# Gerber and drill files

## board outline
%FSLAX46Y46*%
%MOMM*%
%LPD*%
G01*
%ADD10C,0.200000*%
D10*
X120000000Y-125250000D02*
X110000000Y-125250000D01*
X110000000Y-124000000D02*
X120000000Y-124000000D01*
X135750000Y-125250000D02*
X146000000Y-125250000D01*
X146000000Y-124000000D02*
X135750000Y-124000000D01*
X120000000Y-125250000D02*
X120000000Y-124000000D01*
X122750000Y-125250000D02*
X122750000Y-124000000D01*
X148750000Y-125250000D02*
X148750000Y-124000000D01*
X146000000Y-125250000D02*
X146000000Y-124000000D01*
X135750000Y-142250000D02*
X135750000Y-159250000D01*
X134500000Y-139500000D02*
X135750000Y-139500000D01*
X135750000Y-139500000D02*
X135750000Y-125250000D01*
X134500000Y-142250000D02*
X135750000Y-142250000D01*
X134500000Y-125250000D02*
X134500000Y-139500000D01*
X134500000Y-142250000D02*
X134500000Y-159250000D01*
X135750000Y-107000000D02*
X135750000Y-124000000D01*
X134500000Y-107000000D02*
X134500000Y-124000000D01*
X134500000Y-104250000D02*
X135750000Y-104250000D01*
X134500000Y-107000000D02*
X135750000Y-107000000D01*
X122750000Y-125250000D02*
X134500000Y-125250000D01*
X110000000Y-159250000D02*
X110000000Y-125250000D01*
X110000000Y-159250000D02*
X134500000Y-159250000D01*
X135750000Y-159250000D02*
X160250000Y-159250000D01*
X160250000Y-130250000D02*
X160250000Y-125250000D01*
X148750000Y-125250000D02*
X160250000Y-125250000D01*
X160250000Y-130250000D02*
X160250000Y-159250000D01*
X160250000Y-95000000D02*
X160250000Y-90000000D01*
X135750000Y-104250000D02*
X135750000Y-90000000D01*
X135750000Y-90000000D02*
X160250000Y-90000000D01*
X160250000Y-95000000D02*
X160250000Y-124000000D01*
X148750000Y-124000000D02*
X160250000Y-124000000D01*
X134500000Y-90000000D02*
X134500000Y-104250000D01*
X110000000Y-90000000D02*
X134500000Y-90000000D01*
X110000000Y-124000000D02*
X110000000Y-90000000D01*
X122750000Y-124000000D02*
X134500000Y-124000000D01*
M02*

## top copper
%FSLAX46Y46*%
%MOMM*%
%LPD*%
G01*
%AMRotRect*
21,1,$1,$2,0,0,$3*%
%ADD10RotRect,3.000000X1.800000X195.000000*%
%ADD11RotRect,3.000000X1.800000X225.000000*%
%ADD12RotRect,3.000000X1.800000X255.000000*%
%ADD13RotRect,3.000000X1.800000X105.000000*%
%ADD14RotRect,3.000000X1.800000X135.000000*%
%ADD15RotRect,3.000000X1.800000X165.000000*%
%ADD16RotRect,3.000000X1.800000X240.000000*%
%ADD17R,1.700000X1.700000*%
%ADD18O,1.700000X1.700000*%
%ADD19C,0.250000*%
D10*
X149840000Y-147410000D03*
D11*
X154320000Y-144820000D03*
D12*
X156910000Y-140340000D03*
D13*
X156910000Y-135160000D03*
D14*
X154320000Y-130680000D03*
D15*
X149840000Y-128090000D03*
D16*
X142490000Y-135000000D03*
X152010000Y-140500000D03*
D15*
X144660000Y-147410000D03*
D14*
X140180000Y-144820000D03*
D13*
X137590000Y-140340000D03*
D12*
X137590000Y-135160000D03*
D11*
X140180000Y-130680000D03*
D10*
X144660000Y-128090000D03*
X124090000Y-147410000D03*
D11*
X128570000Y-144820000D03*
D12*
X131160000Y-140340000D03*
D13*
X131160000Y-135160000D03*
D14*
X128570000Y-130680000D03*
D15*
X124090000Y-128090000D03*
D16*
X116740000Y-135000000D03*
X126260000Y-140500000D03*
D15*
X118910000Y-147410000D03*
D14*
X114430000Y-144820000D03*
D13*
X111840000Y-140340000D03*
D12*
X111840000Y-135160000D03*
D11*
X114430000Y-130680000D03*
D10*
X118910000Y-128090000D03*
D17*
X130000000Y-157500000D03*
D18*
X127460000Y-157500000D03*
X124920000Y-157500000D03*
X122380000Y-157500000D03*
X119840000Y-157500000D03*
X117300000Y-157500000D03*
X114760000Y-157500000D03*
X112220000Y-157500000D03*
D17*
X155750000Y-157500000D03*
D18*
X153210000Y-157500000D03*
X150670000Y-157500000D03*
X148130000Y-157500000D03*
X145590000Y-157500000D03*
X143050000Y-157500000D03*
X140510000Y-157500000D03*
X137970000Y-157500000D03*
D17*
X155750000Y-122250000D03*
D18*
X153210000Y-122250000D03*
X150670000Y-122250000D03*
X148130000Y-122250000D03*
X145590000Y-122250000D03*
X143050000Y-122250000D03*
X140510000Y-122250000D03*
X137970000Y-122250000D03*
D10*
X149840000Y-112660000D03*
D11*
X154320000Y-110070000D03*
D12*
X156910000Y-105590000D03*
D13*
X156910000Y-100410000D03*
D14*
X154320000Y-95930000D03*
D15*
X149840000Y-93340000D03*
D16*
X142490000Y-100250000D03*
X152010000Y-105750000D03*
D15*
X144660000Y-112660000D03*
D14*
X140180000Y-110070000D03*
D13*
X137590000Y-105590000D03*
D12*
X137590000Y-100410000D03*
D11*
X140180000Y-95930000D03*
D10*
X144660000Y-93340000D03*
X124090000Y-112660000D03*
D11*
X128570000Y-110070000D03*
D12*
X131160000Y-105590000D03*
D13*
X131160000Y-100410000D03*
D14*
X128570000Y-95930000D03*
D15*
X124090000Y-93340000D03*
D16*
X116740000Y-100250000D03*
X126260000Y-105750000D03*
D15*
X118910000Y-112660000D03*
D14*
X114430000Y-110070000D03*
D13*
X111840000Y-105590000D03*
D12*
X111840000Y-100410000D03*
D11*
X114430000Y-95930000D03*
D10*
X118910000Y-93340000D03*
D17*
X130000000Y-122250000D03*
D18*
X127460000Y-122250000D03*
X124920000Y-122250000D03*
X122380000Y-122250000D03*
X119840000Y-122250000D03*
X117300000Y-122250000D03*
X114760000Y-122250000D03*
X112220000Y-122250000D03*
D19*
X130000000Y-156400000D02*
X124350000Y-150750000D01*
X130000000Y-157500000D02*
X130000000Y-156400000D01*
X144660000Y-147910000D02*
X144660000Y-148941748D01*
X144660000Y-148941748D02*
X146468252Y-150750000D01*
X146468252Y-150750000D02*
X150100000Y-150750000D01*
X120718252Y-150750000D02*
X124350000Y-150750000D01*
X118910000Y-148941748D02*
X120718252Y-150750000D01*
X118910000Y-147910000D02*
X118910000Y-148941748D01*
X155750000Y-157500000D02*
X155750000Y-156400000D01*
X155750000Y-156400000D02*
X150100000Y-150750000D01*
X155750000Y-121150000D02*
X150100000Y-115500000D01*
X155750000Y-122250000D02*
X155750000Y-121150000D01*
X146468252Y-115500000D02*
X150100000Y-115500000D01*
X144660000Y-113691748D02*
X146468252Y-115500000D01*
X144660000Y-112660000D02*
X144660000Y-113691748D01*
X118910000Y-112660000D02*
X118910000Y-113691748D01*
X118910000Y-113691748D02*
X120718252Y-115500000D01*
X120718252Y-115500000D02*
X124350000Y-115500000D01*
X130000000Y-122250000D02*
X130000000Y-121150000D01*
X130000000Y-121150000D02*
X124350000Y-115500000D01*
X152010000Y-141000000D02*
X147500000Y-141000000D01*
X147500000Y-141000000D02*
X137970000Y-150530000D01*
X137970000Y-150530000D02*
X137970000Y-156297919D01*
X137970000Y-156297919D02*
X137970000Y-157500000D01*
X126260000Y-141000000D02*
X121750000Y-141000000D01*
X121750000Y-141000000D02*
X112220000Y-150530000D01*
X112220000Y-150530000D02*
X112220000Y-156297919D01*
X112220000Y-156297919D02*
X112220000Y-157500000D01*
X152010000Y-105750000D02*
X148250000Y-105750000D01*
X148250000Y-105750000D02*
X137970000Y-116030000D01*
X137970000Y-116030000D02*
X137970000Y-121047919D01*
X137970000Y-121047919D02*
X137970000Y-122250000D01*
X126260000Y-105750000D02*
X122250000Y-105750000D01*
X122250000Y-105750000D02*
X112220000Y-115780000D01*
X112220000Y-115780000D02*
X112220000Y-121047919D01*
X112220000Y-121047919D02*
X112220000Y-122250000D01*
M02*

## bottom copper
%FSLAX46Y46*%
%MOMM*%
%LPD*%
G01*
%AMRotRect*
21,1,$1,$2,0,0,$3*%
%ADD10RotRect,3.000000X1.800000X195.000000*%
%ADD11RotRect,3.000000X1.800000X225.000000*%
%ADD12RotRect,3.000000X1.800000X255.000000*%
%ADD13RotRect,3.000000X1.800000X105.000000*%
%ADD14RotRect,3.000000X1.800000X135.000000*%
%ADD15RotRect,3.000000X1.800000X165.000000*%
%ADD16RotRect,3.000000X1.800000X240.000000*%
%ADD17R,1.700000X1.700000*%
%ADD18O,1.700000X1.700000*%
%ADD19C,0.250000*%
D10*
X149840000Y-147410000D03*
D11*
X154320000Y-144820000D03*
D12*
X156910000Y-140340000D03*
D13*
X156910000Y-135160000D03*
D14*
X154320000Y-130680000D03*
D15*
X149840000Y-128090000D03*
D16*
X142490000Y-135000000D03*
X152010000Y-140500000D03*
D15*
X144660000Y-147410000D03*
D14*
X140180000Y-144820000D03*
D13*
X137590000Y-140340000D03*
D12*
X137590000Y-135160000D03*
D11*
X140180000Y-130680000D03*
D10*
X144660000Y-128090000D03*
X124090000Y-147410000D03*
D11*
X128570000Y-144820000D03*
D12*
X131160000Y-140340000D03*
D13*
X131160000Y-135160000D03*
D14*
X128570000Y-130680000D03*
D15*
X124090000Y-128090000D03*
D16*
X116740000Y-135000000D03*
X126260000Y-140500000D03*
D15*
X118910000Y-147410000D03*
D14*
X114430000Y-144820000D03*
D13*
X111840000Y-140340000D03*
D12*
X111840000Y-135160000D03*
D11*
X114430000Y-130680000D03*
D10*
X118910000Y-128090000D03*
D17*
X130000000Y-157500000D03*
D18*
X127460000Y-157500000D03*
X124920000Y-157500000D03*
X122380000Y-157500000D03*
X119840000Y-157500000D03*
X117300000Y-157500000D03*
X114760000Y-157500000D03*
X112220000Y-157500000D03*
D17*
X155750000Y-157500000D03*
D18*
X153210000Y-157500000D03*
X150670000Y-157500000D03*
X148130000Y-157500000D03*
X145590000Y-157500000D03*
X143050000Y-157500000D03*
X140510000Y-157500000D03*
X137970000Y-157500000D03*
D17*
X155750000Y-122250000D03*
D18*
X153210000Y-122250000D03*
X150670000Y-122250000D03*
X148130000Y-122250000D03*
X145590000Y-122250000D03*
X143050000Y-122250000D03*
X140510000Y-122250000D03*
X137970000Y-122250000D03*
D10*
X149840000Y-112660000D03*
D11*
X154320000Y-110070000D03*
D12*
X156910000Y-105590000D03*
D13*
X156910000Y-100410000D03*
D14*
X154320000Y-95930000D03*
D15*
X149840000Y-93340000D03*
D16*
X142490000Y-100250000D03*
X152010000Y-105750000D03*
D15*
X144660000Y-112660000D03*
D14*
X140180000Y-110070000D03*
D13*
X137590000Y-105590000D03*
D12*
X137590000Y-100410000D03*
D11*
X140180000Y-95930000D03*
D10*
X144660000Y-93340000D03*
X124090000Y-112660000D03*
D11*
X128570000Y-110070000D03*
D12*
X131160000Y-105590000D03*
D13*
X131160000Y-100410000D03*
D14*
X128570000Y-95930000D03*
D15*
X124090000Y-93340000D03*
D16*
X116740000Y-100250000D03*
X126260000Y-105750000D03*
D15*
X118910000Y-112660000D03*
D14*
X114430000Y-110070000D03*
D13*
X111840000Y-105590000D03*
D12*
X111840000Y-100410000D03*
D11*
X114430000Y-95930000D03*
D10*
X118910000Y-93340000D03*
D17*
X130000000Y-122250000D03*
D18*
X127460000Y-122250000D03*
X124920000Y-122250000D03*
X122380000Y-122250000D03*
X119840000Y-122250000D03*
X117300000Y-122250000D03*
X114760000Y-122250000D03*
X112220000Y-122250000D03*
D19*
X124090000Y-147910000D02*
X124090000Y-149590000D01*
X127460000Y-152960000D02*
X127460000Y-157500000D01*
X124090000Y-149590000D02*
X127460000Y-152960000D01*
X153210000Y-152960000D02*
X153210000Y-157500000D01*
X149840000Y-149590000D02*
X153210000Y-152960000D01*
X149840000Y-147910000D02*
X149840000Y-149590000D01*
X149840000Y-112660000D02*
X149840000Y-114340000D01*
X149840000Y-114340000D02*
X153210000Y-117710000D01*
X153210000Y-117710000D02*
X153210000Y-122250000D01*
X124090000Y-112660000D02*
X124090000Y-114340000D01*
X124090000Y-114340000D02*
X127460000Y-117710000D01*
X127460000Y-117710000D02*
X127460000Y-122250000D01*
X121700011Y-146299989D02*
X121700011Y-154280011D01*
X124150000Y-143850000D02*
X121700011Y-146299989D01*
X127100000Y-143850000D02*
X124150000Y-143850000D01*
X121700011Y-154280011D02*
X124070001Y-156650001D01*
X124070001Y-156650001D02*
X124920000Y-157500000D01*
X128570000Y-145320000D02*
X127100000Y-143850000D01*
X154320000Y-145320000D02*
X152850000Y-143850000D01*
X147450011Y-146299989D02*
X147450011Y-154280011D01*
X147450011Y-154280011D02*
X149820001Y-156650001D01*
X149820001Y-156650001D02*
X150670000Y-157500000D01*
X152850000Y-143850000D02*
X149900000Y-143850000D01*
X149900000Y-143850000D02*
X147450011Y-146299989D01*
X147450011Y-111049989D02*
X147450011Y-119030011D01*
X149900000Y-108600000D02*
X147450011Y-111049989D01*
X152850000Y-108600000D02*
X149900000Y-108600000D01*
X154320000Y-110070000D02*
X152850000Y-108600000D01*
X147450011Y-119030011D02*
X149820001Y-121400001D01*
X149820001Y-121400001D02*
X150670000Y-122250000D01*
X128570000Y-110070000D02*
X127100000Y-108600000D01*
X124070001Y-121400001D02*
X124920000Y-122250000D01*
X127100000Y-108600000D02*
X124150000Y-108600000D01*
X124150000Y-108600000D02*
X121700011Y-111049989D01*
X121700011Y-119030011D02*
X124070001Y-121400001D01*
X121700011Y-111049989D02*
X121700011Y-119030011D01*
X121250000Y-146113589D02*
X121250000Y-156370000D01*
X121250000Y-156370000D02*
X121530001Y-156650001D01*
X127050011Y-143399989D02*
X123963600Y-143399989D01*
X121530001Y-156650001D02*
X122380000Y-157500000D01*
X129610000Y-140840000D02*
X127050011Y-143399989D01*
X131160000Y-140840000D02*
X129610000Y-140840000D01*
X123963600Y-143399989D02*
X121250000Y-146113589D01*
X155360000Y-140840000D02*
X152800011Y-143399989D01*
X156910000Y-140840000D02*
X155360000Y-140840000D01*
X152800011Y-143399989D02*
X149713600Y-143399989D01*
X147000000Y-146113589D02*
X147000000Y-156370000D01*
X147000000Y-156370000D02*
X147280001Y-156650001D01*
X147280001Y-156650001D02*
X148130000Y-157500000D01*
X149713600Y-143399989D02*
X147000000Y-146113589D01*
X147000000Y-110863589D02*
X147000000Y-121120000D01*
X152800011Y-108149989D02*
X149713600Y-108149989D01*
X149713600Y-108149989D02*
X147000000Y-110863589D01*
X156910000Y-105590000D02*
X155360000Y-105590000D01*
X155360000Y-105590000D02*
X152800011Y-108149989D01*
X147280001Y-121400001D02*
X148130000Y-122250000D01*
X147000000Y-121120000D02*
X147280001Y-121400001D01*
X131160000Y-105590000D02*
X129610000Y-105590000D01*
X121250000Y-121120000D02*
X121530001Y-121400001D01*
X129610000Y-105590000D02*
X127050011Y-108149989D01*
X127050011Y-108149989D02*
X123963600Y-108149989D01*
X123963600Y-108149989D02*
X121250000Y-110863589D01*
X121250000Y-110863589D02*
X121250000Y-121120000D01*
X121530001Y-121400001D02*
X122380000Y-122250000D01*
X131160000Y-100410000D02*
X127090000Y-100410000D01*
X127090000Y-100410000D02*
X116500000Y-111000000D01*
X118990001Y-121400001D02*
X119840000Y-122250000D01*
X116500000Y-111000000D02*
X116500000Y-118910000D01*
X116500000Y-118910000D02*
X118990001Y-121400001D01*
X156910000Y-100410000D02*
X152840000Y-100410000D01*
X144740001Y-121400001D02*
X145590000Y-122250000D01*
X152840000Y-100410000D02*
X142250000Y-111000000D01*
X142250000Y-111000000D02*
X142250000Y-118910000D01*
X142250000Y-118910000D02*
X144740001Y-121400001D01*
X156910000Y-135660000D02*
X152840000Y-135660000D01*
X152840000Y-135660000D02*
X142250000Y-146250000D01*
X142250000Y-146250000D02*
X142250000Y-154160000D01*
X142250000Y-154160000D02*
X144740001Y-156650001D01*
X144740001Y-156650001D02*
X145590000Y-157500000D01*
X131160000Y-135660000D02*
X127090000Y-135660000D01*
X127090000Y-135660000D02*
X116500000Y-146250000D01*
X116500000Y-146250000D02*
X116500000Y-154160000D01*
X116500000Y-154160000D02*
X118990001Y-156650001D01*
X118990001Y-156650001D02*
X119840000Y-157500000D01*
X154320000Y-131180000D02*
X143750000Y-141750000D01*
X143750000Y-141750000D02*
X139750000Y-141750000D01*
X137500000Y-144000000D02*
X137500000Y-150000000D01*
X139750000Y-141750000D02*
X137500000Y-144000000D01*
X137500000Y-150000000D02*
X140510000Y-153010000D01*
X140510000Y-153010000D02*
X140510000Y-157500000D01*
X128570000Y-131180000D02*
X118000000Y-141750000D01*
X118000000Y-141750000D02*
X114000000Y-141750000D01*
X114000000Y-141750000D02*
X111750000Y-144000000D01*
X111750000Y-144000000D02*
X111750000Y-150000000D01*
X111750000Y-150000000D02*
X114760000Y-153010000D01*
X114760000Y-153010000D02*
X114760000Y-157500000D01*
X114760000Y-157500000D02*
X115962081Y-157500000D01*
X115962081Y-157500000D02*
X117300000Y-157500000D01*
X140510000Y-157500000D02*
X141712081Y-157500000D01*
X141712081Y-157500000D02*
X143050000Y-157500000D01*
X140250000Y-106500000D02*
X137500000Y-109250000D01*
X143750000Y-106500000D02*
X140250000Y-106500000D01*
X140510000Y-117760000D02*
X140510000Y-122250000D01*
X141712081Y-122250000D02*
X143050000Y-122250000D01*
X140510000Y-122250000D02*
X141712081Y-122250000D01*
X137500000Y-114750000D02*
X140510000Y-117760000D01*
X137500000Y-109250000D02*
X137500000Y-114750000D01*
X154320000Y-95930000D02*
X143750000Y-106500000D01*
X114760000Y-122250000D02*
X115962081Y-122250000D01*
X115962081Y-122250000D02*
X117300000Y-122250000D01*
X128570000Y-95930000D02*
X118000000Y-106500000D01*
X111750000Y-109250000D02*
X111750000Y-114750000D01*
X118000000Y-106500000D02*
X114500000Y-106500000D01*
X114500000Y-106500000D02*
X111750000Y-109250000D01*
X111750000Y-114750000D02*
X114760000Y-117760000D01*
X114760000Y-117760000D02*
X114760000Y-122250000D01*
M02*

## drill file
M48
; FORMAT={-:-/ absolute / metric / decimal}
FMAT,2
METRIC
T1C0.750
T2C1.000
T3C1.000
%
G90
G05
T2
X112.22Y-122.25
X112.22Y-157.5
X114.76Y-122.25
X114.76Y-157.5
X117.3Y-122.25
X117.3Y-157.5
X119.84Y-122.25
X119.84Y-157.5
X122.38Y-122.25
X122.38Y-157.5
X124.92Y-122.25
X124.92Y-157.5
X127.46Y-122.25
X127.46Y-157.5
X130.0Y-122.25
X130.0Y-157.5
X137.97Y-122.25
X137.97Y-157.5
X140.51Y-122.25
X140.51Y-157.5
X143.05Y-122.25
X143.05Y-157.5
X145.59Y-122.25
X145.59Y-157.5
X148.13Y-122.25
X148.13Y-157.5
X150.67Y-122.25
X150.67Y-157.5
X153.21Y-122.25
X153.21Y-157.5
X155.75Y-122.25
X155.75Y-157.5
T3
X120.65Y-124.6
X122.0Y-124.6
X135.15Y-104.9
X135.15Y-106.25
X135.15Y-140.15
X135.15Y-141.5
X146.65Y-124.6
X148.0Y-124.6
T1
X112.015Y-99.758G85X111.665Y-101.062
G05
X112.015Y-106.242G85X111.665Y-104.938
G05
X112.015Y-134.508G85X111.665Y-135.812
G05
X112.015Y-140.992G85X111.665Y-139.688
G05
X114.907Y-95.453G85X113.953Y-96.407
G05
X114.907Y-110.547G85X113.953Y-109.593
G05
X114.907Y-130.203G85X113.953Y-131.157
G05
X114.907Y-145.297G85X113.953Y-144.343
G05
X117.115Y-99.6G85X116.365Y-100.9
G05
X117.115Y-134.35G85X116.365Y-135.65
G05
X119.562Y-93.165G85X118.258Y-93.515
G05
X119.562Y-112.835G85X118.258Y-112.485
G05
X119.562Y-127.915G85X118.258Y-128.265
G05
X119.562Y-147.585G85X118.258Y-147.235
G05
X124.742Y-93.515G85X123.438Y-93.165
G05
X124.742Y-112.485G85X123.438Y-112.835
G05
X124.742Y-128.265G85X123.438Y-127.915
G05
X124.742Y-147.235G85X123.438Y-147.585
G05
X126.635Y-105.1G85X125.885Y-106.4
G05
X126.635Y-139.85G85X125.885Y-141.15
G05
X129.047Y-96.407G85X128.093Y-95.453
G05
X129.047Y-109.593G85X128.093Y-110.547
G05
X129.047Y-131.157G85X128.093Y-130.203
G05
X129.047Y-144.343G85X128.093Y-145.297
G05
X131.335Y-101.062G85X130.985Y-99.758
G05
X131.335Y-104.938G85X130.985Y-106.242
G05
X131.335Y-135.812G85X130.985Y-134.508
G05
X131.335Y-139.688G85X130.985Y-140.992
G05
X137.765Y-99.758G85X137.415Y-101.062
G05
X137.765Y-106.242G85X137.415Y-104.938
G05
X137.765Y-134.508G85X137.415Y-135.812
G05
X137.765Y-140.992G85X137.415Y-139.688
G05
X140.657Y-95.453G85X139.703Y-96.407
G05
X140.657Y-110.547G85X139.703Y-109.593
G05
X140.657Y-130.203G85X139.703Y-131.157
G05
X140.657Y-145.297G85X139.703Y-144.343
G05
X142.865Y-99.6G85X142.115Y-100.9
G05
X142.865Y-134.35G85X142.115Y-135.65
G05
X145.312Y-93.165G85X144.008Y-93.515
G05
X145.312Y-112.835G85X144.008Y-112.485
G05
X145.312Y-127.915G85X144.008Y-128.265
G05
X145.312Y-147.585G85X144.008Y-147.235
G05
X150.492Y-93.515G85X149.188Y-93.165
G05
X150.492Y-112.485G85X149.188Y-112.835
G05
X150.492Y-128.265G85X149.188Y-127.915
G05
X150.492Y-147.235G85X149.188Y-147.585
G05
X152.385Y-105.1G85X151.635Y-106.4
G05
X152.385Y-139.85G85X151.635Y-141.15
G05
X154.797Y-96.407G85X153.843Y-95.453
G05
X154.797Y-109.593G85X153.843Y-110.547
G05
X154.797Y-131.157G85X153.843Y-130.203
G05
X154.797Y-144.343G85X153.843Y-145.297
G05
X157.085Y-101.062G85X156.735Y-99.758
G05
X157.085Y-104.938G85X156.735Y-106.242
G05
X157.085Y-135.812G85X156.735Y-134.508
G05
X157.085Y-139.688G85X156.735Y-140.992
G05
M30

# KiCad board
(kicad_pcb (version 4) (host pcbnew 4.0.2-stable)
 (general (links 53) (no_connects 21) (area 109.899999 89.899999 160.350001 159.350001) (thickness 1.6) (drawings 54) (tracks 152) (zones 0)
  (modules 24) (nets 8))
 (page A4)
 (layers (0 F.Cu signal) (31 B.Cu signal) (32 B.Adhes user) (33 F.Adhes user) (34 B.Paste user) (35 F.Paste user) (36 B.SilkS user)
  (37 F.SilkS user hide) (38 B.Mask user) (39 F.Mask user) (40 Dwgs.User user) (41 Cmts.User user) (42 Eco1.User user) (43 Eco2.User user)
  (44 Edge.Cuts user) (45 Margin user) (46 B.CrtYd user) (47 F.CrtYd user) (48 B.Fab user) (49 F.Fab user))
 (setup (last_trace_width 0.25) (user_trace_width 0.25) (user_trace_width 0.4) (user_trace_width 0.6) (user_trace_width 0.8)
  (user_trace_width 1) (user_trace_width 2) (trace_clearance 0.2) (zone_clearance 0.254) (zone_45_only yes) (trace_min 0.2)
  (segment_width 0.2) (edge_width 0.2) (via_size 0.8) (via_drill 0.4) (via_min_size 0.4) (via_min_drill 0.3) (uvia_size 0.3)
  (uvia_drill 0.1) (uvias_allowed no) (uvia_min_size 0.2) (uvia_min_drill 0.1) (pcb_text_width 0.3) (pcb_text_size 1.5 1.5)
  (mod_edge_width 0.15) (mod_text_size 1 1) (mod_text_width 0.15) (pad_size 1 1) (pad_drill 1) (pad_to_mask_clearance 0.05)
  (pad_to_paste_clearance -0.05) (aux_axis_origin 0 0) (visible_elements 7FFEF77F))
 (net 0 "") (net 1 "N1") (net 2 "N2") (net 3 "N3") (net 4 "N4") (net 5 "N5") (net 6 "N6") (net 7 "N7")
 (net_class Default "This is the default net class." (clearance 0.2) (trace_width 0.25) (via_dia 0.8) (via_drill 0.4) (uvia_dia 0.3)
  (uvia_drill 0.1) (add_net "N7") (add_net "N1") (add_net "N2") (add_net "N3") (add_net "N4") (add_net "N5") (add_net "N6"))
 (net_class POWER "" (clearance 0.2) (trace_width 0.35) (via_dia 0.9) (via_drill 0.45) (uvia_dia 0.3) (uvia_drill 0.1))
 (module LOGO (layer B.Cu) (at 146.55 102.95 180)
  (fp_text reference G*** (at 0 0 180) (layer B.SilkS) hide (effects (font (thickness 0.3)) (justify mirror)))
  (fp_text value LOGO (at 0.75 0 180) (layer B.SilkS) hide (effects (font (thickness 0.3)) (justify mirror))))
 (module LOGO (layer B.Cu) (at 120.75 102.95 180)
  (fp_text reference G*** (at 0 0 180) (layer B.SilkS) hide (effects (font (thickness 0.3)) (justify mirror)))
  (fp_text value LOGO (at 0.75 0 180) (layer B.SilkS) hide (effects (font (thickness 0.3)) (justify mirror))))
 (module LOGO (layer B.Cu) (at 120.74759 137.777062 180)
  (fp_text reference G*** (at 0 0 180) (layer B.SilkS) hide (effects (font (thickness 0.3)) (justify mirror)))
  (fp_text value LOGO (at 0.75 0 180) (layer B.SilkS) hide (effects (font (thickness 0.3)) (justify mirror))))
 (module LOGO (layer B.Cu) (at 146.59759 137.777062 180)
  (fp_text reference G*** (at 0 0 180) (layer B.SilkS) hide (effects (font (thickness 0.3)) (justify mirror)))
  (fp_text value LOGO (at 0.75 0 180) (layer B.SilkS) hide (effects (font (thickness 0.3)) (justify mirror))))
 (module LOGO (layer F.Cu) (at 121.5 137.75 285)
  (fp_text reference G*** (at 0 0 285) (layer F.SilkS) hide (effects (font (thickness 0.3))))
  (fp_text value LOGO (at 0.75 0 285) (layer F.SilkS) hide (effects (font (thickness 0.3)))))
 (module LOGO (layer F.Cu) (at 147.25 137.75 285)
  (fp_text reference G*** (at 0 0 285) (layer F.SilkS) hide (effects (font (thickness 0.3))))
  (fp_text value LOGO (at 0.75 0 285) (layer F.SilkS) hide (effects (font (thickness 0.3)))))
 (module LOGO (layer F.Cu) (at 147.25 103 285)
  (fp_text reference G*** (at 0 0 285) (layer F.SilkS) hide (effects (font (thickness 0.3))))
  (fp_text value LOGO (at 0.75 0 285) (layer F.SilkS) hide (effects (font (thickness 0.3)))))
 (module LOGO (layer F.Cu) (at 121.5 103 285)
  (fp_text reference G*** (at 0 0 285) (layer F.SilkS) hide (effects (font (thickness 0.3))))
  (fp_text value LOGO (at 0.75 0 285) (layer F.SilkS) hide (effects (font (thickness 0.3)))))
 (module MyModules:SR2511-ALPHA (layer F.Cu) (at 147.25 137.75 180)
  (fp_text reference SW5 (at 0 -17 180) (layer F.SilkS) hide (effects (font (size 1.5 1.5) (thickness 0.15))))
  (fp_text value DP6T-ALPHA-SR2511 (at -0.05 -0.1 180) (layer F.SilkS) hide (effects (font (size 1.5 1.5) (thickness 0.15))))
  (pad 1 thru_hole rect (at -2.59 -9.66 195) (size 3 1.8) (drill oval 2.1 0.75) (layers *.Cu *.Mask F.SilkS) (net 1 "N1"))
  (pad 12 thru_hole rect (at -7.07 -7.07 225) (size 3 1.8) (drill oval 2.1 0.75) (layers *.Cu *.Mask F.SilkS) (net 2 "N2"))
  (pad 11 thru_hole rect (at -9.66 -2.59 255) (size 3 1.8) (drill oval 2.1 0.75) (layers *.Cu *.Mask F.SilkS) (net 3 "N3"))
  (pad 10 thru_hole rect (at -9.66 2.59 105) (size 3 1.8) (drill oval 2.1 0.75) (layers *.Cu *.Mask F.SilkS) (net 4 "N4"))
  (pad 9 thru_hole rect (at -7.07 7.07 135) (size 3 1.8) (drill oval 2.1 0.75) (layers *.Cu *.Mask F.SilkS) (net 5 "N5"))
  (pad 8 thru_hole rect (at -2.59 9.66 165) (size 3 1.8) (drill oval 2.1 0.75) (layers *.Cu *.Mask F.SilkS))
  (pad D thru_hole rect (at 4.76 2.75 240) (size 3 1.8) (drill oval 2.25 0.75) (layers *.Cu *.Mask F.SilkS))
  (pad A thru_hole rect (at -4.76 -2.75 240) (size 3 1.8) (drill oval 2.25 0.75) (layers *.Cu *.Mask F.SilkS) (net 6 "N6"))
  (pad 2 thru_hole rect (at 2.59 -9.66 165) (size 3 1.8) (drill oval 2.1 0.75) (layers *.Cu *.Mask F.SilkS) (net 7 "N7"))
  (pad 3 thru_hole rect (at 7.07 -7.07 135) (size 3 1.8) (drill oval 2.1 0.75) (layers *.Cu *.Mask F.SilkS))
  (pad 4 thru_hole rect (at 9.66 -2.59 105) (size 3 1.8) (drill oval 2.1 0.75) (layers *.Cu *.Mask F.SilkS))
  (pad 5 thru_hole rect (at 9.66 2.59 255) (size 3 1.8) (drill oval 2.1 0.75) (layers *.Cu *.Mask F.SilkS))
  (pad 6 thru_hole rect (at 7.07 7.07 225) (size 3 1.8) (drill oval 2.1 0.75) (layers *.Cu *.Mask F.SilkS))
  (pad 7 thru_hole rect (at 2.59 9.66 195) (size 3 1.8) (drill oval 2.1 0.75) (layers *.Cu *.Mask F.SilkS)))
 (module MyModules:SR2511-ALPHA (layer F.Cu) (at 121.5 137.75 180)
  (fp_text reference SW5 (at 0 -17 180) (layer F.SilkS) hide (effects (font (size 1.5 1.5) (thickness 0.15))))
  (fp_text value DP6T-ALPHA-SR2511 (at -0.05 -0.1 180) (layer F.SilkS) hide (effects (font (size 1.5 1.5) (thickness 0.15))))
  (pad 1 thru_hole rect (at -2.59 -9.66 195) (size 3 1.8) (drill oval 2.1 0.75) (layers *.Cu *.Mask F.SilkS) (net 1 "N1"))
  (pad 12 thru_hole rect (at -7.07 -7.07 225) (size 3 1.8) (drill oval 2.1 0.75) (layers *.Cu *.Mask F.SilkS) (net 2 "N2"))
  (pad 11 thru_hole rect (at -9.66 -2.59 255) (size 3 1.8) (drill oval 2.1 0.75) (layers *.Cu *.Mask F.SilkS) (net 3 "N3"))
  (pad 10 thru_hole rect (at -9.66 2.59 105) (size 3 1.8) (drill oval 2.1 0.75) (layers *.Cu *.Mask F.SilkS) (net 4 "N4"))
  (pad 9 thru_hole rect (at -7.07 7.07 135) (size 3 1.8) (drill oval 2.1 0.75) (layers *.Cu *.Mask F.SilkS) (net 5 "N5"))
  (pad 8 thru_hole rect (at -2.59 9.66 165) (size 3 1.8) (drill oval 2.1 0.75) (layers *.Cu *.Mask F.SilkS))
  (pad D thru_hole rect (at 4.76 2.75 240) (size 3 1.8) (drill oval 2.25 0.75) (layers *.Cu *.Mask F.SilkS))
  (pad A thru_hole rect (at -4.76 -2.75 240) (size 3 1.8) (drill oval 2.25 0.75) (layers *.Cu *.Mask F.SilkS) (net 6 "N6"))
  (pad 2 thru_hole rect (at 2.59 -9.66 165) (size 3 1.8) (drill oval 2.1 0.75) (layers *.Cu *.Mask F.SilkS) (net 7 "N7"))
  (pad 3 thru_hole rect (at 7.07 -7.07 135) (size 3 1.8) (drill oval 2.1 0.75) (layers *.Cu *.Mask F.SilkS))
  (pad 4 thru_hole rect (at 9.66 -2.59 105) (size 3 1.8) (drill oval 2.1 0.75) (layers *.Cu *.Mask F.SilkS))
  (pad 5 thru_hole rect (at 9.66 2.59 255) (size 3 1.8) (drill oval 2.1 0.75) (layers *.Cu *.Mask F.SilkS))
  (pad 6 thru_hole rect (at 7.07 7.07 225) (size 3 1.8) (drill oval 2.1 0.75) (layers *.Cu *.Mask F.SilkS))
  (pad 7 thru_hole rect (at 2.59 9.66 195) (size 3 1.8) (drill oval 2.1 0.75) (layers *.Cu *.Mask F.SilkS)))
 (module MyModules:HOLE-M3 (layer F.Cu) (at 122 124.6 90)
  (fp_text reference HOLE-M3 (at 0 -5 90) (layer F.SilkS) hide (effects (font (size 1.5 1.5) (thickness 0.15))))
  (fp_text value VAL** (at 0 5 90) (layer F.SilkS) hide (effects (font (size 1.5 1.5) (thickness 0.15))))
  (pad "" np_thru_hole circle (at 0 0 90) (size 1 1) (drill 1) (layers *.Cu *.Mask F.SilkS)))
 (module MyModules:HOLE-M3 (layer F.Cu) (at 120.65 124.6 90)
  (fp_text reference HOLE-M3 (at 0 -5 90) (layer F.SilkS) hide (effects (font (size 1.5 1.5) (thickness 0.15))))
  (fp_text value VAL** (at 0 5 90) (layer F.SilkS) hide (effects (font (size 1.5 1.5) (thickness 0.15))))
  (pad "" np_thru_hole circle (at 0 0 90) (size 1 1) (drill 1) (layers *.Cu *.Mask F.SilkS)))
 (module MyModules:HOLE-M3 (layer F.Cu) (at 146.65 124.6 90)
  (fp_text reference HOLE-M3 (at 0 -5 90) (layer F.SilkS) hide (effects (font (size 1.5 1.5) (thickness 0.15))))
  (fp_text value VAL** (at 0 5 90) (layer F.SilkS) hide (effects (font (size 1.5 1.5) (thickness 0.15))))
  (pad "" np_thru_hole circle (at 0 0 90) (size 1 1) (drill 1) (layers *.Cu *.Mask F.SilkS)))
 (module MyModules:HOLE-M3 (layer F.Cu) (at 148 124.6 90)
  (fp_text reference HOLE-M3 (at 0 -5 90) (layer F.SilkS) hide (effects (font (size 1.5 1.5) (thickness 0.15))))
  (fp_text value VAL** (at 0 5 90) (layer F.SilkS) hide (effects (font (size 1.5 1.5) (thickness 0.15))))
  (pad "" np_thru_hole circle (at 0 0 90) (size 1 1) (drill 1) (layers *.Cu *.Mask F.SilkS)))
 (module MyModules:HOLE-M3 (layer F.Cu) (at 135.15 141.5)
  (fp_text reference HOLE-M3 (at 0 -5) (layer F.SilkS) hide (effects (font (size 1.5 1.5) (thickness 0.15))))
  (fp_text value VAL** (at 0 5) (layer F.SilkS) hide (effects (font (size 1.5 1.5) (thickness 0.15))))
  (pad "" np_thru_hole circle (at 0 0) (size 1 1) (drill 1) (layers *.Cu *.Mask F.SilkS)))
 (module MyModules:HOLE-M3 (layer F.Cu) (at 135.15 140.15)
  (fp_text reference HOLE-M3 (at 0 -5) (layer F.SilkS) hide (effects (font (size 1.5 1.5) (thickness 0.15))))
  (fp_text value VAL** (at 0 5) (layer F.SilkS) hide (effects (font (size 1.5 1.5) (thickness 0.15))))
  (pad "" np_thru_hole circle (at 0 0) (size 1 1) (drill 1) (layers *.Cu *.Mask F.SilkS)))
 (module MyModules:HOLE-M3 (layer F.Cu) (at 135.15 106.25)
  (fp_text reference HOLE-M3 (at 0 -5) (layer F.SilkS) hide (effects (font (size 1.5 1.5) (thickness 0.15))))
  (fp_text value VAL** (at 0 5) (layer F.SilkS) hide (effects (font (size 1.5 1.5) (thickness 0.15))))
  (pad "" np_thru_hole circle (at 0 0) (size 1 1) (drill 1) (layers *.Cu *.Mask F.SilkS)))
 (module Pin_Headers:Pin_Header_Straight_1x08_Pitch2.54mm (layer F.Cu) (at 130 157.5 270)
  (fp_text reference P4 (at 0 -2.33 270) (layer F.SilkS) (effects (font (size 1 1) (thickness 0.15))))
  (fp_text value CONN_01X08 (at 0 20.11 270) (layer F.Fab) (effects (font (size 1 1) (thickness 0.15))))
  (pad 1 thru_hole rect (at 0 0 270) (size 1.7 1.7) (drill 1) (layers *.Cu *.Mask) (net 7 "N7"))
  (pad 2 thru_hole oval (at 0 2.54 270) (size 1.7 1.7) (drill 1) (layers *.Cu *.Mask) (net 1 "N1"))
  (pad 3 thru_hole oval (at 0 5.08 270) (size 1.7 1.7) (drill 1) (layers *.Cu *.Mask) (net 2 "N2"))
  (pad 4 thru_hole oval (at 0 7.62 270) (size 1.7 1.7) (drill 1) (layers *.Cu *.Mask) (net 3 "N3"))
  (pad 5 thru_hole oval (at 0 10.16 270) (size 1.7 1.7) (drill 1) (layers *.Cu *.Mask) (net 4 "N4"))
  (pad 6 thru_hole oval (at 0 12.7 270) (size 1.7 1.7) (drill 1) (layers *.Cu *.Mask) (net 5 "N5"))
  (pad 7 thru_hole oval (at 0 15.24 270) (size 1.7 1.7) (drill 1) (layers *.Cu *.Mask) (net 5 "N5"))
  (pad 8 thru_hole oval (at 0 17.78 270) (size 1.7 1.7) (drill 1) (layers *.Cu *.Mask) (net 6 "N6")))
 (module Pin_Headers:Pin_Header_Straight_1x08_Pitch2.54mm (layer F.Cu) (at 155.75 157.5 270)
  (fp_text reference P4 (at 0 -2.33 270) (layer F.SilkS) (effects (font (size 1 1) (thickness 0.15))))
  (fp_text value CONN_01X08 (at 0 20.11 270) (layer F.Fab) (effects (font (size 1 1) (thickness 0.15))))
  (pad 1 thru_hole rect (at 0 0 270) (size 1.7 1.7) (drill 1) (layers *.Cu *.Mask) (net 7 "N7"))
  (pad 2 thru_hole oval (at 0 2.54 270) (size 1.7 1.7) (drill 1) (layers *.Cu *.Mask) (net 1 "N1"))
  (pad 3 thru_hole oval (at 0 5.08 270) (size 1.7 1.7) (drill 1) (layers *.Cu *.Mask) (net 2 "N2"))
  (pad 4 thru_hole oval (at 0 7.62 270) (size 1.7 1.7) (drill 1) (layers *.Cu *.Mask) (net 3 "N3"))
  (pad 5 thru_hole oval (at 0 10.16 270) (size 1.7 1.7) (drill 1) (layers *.Cu *.Mask) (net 4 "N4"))
  (pad 6 thru_hole oval (at 0 12.7 270) (size 1.7 1.7) (drill 1) (layers *.Cu *.Mask) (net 5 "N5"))
  (pad 7 thru_hole oval (at 0 15.24 270) (size 1.7 1.7) (drill 1) (layers *.Cu *.Mask) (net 5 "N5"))
  (pad 8 thru_hole oval (at 0 17.78 270) (size 1.7 1.7) (drill 1) (layers *.Cu *.Mask) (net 6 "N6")))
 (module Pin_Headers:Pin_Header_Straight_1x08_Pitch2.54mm (layer F.Cu) (at 155.75 122.25 270)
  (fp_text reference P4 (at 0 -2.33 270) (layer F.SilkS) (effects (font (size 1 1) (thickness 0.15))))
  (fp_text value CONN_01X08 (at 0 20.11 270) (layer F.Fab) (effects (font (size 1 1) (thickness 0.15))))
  (pad 1 thru_hole rect (at 0 0 270) (size 1.7 1.7) (drill 1) (layers *.Cu *.Mask) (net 7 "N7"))
  (pad 2 thru_hole oval (at 0 2.54 270) (size 1.7 1.7) (drill 1) (layers *.Cu *.Mask) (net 1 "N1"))
  (pad 3 thru_hole oval (at 0 5.08 270) (size 1.7 1.7) (drill 1) (layers *.Cu *.Mask) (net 2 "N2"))
  (pad 4 thru_hole oval (at 0 7.62 270) (size 1.7 1.7) (drill 1) (layers *.Cu *.Mask) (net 3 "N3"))
  (pad 5 thru_hole oval (at 0 10.16 270) (size 1.7 1.7) (drill 1) (layers *.Cu *.Mask) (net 4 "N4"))
  (pad 6 thru_hole oval (at 0 12.7 270) (size 1.7 1.7) (drill 1) (layers *.Cu *.Mask) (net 5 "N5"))
  (pad 7 thru_hole oval (at 0 15.24 270) (size 1.7 1.7) (drill 1) (layers *.Cu *.Mask) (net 5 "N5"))
  (pad 8 thru_hole oval (at 0 17.78 270) (size 1.7 1.7) (drill 1) (layers *.Cu *.Mask) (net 6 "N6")))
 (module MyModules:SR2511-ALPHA (layer F.Cu) (at 147.25 103 180)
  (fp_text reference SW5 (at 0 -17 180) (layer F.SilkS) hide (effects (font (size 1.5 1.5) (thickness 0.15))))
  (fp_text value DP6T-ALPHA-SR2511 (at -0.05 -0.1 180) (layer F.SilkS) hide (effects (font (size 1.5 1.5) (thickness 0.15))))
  (pad 1 thru_hole rect (at -2.59 -9.66 195) (size 3 1.8) (drill oval 2.1 0.75) (layers *.Cu *.Mask F.SilkS) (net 1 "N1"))
  (pad 12 thru_hole rect (at -7.07 -7.07 225) (size 3 1.8) (drill oval 2.1 0.75) (layers *.Cu *.Mask F.SilkS) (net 2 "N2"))
  (pad 11 thru_hole rect (at -9.66 -2.59 255) (size 3 1.8) (drill oval 2.1 0.75) (layers *.Cu *.Mask F.SilkS) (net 3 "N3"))
  (pad 10 thru_hole rect (at -9.66 2.59 105) (size 3 1.8) (drill oval 2.1 0.75) (layers *.Cu *.Mask F.SilkS) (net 4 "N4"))
  (pad 9 thru_hole rect (at -7.07 7.07 135) (size 3 1.8) (drill oval 2.1 0.75) (layers *.Cu *.Mask F.SilkS) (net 5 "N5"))
  (pad 8 thru_hole rect (at -2.59 9.66 165) (size 3 1.8) (drill oval 2.1 0.75) (layers *.Cu *.Mask F.SilkS))
  (pad D thru_hole rect (at 4.76 2.75 240) (size 3 1.8) (drill oval 2.25 0.75) (layers *.Cu *.Mask F.SilkS))
  (pad A thru_hole rect (at -4.76 -2.75 240) (size 3 1.8) (drill oval 2.25 0.75) (layers *.Cu *.Mask F.SilkS) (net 6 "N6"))
  (pad 2 thru_hole rect (at 2.59 -9.66 165) (size 3 1.8) (drill oval 2.1 0.75) (layers *.Cu *.Mask F.SilkS) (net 7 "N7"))
  (pad 3 thru_hole rect (at 7.07 -7.07 135) (size 3 1.8) (drill oval 2.1 0.75) (layers *.Cu *.Mask F.SilkS))
  (pad 4 thru_hole rect (at 9.66 -2.59 105) (size 3 1.8) (drill oval 2.1 0.75) (layers *.Cu *.Mask F.SilkS))
  (pad 5 thru_hole rect (at 9.66 2.59 255) (size 3 1.8) (drill oval 2.1 0.75) (layers *.Cu *.Mask F.SilkS))
  (pad 6 thru_hole rect (at 7.07 7.07 225) (size 3 1.8) (drill oval 2.1 0.75) (layers *.Cu *.Mask F.SilkS))
  (pad 7 thru_hole rect (at 2.59 9.66 195) (size 3 1.8) (drill oval 2.1 0.75) (layers *.Cu *.Mask F.SilkS)))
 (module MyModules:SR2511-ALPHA (layer F.Cu) (at 121.5 103 180)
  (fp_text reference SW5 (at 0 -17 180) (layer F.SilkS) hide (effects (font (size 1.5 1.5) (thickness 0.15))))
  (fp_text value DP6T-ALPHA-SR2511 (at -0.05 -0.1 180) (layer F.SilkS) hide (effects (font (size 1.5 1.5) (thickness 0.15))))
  (pad 1 thru_hole rect (at -2.59 -9.66 195) (size 3 1.8) (drill oval 2.1 0.75) (layers *.Cu *.Mask F.SilkS) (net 1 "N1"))
  (pad 12 thru_hole rect (at -7.07 -7.07 225) (size 3 1.8) (drill oval 2.1 0.75) (layers *.Cu *.Mask F.SilkS) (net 2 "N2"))
  (pad 11 thru_hole rect (at -9.66 -2.59 255) (size 3 1.8) (drill oval 2.1 0.75) (layers *.Cu *.Mask F.SilkS) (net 3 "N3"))
  (pad 10 thru_hole rect (at -9.66 2.59 105) (size 3 1.8) (drill oval 2.1 0.75) (layers *.Cu *.Mask F.SilkS) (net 4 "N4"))
  (pad 9 thru_hole rect (at -7.07 7.07 135) (size 3 1.8) (drill oval 2.1 0.75) (layers *.Cu *.Mask F.SilkS) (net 5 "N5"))
  (pad 8 thru_hole rect (at -2.59 9.66 165) (size 3 1.8) (drill oval 2.1 0.75) (layers *.Cu *.Mask F.SilkS))
  (pad D thru_hole rect (at 4.76 2.75 240) (size 3 1.8) (drill oval 2.25 0.75) (layers *.Cu *.Mask F.SilkS))
  (pad A thru_hole rect (at -4.76 -2.75 240) (size 3 1.8) (drill oval 2.25 0.75) (layers *.Cu *.Mask F.SilkS) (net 6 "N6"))
  (pad 2 thru_hole rect (at 2.59 -9.66 165) (size 3 1.8) (drill oval 2.1 0.75) (layers *.Cu *.Mask F.SilkS) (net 7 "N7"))
  (pad 3 thru_hole rect (at 7.07 -7.07 135) (size 3 1.8) (drill oval 2.1 0.75) (layers *.Cu *.Mask F.SilkS))
  (pad 4 thru_hole rect (at 9.66 -2.59 105) (size 3 1.8) (drill oval 2.1 0.75) (layers *.Cu *.Mask F.SilkS))
  (pad 5 thru_hole rect (at 9.66 2.59 255) (size 3 1.8) (drill oval 2.1 0.75) (layers *.Cu *.Mask F.SilkS))
  (pad 6 thru_hole rect (at 7.07 7.07 225) (size 3 1.8) (drill oval 2.1 0.75) (layers *.Cu *.Mask F.SilkS))
  (pad 7 thru_hole rect (at 2.59 9.66 195) (size 3 1.8) (drill oval 2.1 0.75) (layers *.Cu *.Mask F.SilkS)))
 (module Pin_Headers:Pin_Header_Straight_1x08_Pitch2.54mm (layer F.Cu) (at 130 122.25 270)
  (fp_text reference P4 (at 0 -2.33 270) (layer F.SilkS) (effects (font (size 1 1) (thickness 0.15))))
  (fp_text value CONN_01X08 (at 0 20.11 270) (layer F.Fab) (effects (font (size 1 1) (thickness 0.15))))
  (pad 1 thru_hole rect (at 0 0 270) (size 1.7 1.7) (drill 1) (layers *.Cu *.Mask) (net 7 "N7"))
  (pad 2 thru_hole oval (at 0 2.54 270) (size 1.7 1.7) (drill 1) (layers *.Cu *.Mask) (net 1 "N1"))
  (pad 3 thru_hole oval (at 0 5.08 270) (size 1.7 1.7) (drill 1) (layers *.Cu *.Mask) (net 2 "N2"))
  (pad 4 thru_hole oval (at 0 7.62 270) (size 1.7 1.7) (drill 1) (layers *.Cu *.Mask) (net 3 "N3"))
  (pad 5 thru_hole oval (at 0 10.16 270) (size 1.7 1.7) (drill 1) (layers *.Cu *.Mask) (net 4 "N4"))
  (pad 6 thru_hole oval (at 0 12.7 270) (size 1.7 1.7) (drill 1) (layers *.Cu *.Mask) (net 5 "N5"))
  (pad 7 thru_hole oval (at 0 15.24 270) (size 1.7 1.7) (drill 1) (layers *.Cu *.Mask) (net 5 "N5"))
  (pad 8 thru_hole oval (at 0 17.78 270) (size 1.7 1.7) (drill 1) (layers *.Cu *.Mask) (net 6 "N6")))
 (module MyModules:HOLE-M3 (layer F.Cu) (at 135.15 104.9)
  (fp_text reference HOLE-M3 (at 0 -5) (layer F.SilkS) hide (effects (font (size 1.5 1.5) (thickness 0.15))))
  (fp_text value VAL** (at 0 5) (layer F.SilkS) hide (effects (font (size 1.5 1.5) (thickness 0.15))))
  (pad "" np_thru_hole circle (at 0 0) (size 1 1) (drill 1) (layers *.Cu *.Mask F.SilkS)))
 (gr_line (start 120 125.25) (end 110 125.25) (layer Edge.Cuts) (width 0.2))
 (gr_line (start 110 124) (end 120 124) (layer Edge.Cuts) (width 0.2))
 (gr_line (start 135.75 125.25) (end 146 125.25) (layer Edge.Cuts) (width 0.2))
 (gr_line (start 146 124) (end 135.75 124) (layer Edge.Cuts) (width 0.2))
 (gr_line (start 120 125.25) (end 120 124) (layer Edge.Cuts) (width 0.2))
 (gr_line (start 122.75 125.25) (end 122.75 124) (layer Edge.Cuts) (width 0.2))
 (gr_line (start 148.75 125.25) (end 148.75 124) (layer Edge.Cuts) (width 0.2))
 (gr_line (start 146 125.25) (end 146 124) (layer Edge.Cuts) (width 0.2))
 (gr_line (start 135.75 142.25) (end 135.75 159.25) (layer Edge.Cuts) (width 0.2))
 (gr_line (start 134.5 139.5) (end 135.75 139.5) (layer Edge.Cuts) (width 0.2))
 (gr_line (start 135.75 139.5) (end 135.75 125.25) (layer Edge.Cuts) (width 0.2))
 (gr_line (start 134.5 142.25) (end 135.75 142.25) (layer Edge.Cuts) (width 0.2))
 (gr_line (start 134.5 125.25) (end 134.5 139.5) (layer Edge.Cuts) (width 0.2))
 (gr_line (start 134.5 142.25) (end 134.5 159.25) (layer Edge.Cuts) (width 0.2))
 (gr_line (start 135.75 107) (end 135.75 124) (layer Edge.Cuts) (width 0.2))
 (gr_line (start 134.5 107) (end 134.5 124) (layer Edge.Cuts) (width 0.2))
 (gr_line (start 134.5 104.25) (end 135.75 104.25) (layer Edge.Cuts) (width 0.2))
 (gr_line (start 134.5 107) (end 135.75 107) (layer Edge.Cuts) (width 0.2))
 (gr_line (start 122.75 125.25) (end 134.5 125.25) (layer Edge.Cuts) (width 0.2))
 (gr_line (start 110 159.25) (end 110 125.25) (layer Edge.Cuts) (width 0.2))
 (gr_line (start 110 159.25) (end 134.5 159.25) (layer Edge.Cuts) (width 0.2))
 (gr_line (start 135.75 159.25) (end 160.25 159.25) (layer Edge.Cuts) (width 0.2))
 (gr_line (start 160.25 130.25) (end 160.25 125.25) (layer Edge.Cuts) (width 0.2))
 (gr_line (start 148.75 125.25) (end 160.25 125.25) (layer Edge.Cuts) (width 0.2))
 (gr_line (start 160.25 130.25) (end 160.25 159.25) (layer Edge.Cuts) (width 0.2))
 (gr_line (start 160.25 95) (end 160.25 90) (layer Edge.Cuts) (width 0.2))
 (gr_line (start 135.75 104.25) (end 135.75 90) (layer Edge.Cuts) (width 0.2))
 (gr_line (start 135.75 90) (end 160.25 90) (layer Edge.Cuts) (width 0.2))
 (gr_line (start 160.25 95) (end 160.25 124) (layer Edge.Cuts) (width 0.2))
 (gr_line (start 148.75 124) (end 160.25 124) (layer Edge.Cuts) (width 0.2))
 (gr_line (start 134.5 90) (end 134.5 104.25) (layer Edge.Cuts) (width 0.2))
 (gr_line (start 110 90) (end 134.5 90) (layer Edge.Cuts) (width 0.2))
 (gr_line (start 110 124) (end 110 90) (layer Edge.Cuts) (width 0.2))
 (gr_line (start 122.75 124) (end 134.5 124) (layer Edge.Cuts) (width 0.2))
 (segment (start 130 156.4) (end 124.35 150.75) (width 0.25) (layer F.Cu) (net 7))
 (segment (start 130 157.5) (end 130 156.4) (width 0.25) (layer F.Cu) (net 7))
 (segment (start 144.66 147.91) (end 144.66 148.941748) (width 0.25) (layer F.Cu) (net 7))
 (segment (start 144.66 148.941748) (end 146.468252 150.75) (width 0.25) (layer F.Cu) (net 7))
 (segment (start 146.468252 150.75) (end 150.1 150.75) (width 0.25) (layer F.Cu) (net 7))
 (segment (start 120.718252 150.75) (end 124.35 150.75) (width 0.25) (layer F.Cu) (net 7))
 (segment (start 118.91 148.941748) (end 120.718252 150.75) (width 0.25) (layer F.Cu) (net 7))
 (segment (start 118.91 147.91) (end 118.91 148.941748) (width 0.25) (layer F.Cu) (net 7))
 (segment (start 155.75 157.5) (end 155.75 156.4) (width 0.25) (layer F.Cu) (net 7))
 (segment (start 155.75 156.4) (end 150.1 150.75) (width 0.25) (layer F.Cu) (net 7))
 (segment (start 155.75 121.15) (end 150.1 115.5) (width 0.25) (layer F.Cu) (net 7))
 (segment (start 155.75 122.25) (end 155.75 121.15) (width 0.25) (layer F.Cu) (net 7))
 (segment (start 146.468252 115.5) (end 150.1 115.5) (width 0.25) (layer F.Cu) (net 7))
 (segment (start 144.66 113.691748) (end 146.468252 115.5) (width 0.25) (layer F.Cu) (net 7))
 (segment (start 144.66 112.66) (end 144.66 113.691748) (width 0.25) (layer F.Cu) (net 7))
 (segment (start 118.91 112.66) (end 118.91 113.691748) (width 0.25) (layer F.Cu) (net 7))
 (segment (start 118.91 113.691748) (end 120.718252 115.5) (width 0.25) (layer F.Cu) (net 7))
 (segment (start 120.718252 115.5) (end 124.35 115.5) (width 0.25) (layer F.Cu) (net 7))
 (segment (start 130 122.25) (end 130 121.15) (width 0.25) (layer F.Cu) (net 7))
 (segment (start 130 121.15) (end 124.35 115.5) (width 0.25) (layer F.Cu) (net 7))
 (segment (start 124.09 147.91) (end 124.09 149.59) (width 0.25) (layer B.Cu) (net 1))
 (segment (start 127.46 152.96) (end 127.46 157.5) (width 0.25) (layer B.Cu) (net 1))
 (segment (start 124.09 149.59) (end 127.46 152.96) (width 0.25) (layer B.Cu) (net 1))
 (segment (start 153.21 152.96) (end 153.21 157.5) (width 0.25) (layer B.Cu) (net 1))
 (segment (start 149.84 149.59) (end 153.21 152.96) (width 0.25) (layer B.Cu) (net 1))
 (segment (start 149.84 147.91) (end 149.84 149.59) (width 0.25) (layer B.Cu) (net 1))
 (segment (start 149.84 112.66) (end 149.84 114.34) (width 0.25) (layer B.Cu) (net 1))
 (segment (start 149.84 114.34) (end 153.21 117.71) (width 0.25) (layer B.Cu) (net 1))
 (segment (start 153.21 117.71) (end 153.21 122.25) (width 0.25) (layer B.Cu) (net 1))
 (segment (start 124.09 112.66) (end 124.09 114.34) (width 0.25) (layer B.Cu) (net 1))
 (segment (start 124.09 114.34) (end 127.46 117.71) (width 0.25) (layer B.Cu) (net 1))
 (segment (start 127.46 117.71) (end 127.46 122.25) (width 0.25) (layer B.Cu) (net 1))
 (segment (start 121.700011 146.299989) (end 121.700011 154.280011) (width 0.25) (layer B.Cu) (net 2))
 (segment (start 124.15 143.85) (end 121.700011 146.299989) (width 0.25) (layer B.Cu) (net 2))
 (segment (start 127.1 143.85) (end 124.15 143.85) (width 0.25) (layer B.Cu) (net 2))
 (segment (start 121.700011 154.280011) (end 124.070001 156.650001) (width 0.25) (layer B.Cu) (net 2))
 (segment (start 124.070001 156.650001) (end 124.92 157.5) (width 0.25) (layer B.Cu) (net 2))
 (segment (start 128.57 145.32) (end 127.1 143.85) (width 0.25) (layer B.Cu) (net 2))
 (segment (start 154.32 145.32) (end 152.85 143.85) (width 0.25) (layer B.Cu) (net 2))
 (segment (start 147.450011 146.299989) (end 147.450011 154.280011) (width 0.25) (layer B.Cu) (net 2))
 (segment (start 147.450011 154.280011) (end 149.820001 156.650001) (width 0.25) (layer B.Cu) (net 2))
 (segment (start 149.820001 156.650001) (end 150.67 157.5) (width 0.25) (layer B.Cu) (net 2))
 (segment (start 152.85 143.85) (end 149.9 143.85) (width 0.25) (layer B.Cu) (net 2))
 (segment (start 149.9 143.85) (end 147.450011 146.299989) (width 0.25) (layer B.Cu) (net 2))
 (segment (start 147.450011 111.049989) (end 147.450011 119.030011) (width 0.25) (layer B.Cu) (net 2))
 (segment (start 149.9 108.6) (end 147.450011 111.049989) (width 0.25) (layer B.Cu) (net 2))
 (segment (start 152.85 108.6) (end 149.9 108.6) (width 0.25) (layer B.Cu) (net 2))
 (segment (start 154.32 110.07) (end 152.85 108.6) (width 0.25) (layer B.Cu) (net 2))
 (segment (start 147.450011 119.030011) (end 149.820001 121.400001) (width 0.25) (layer B.Cu) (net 2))
 (segment (start 149.820001 121.400001) (end 150.67 122.25) (width 0.25) (layer B.Cu) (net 2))
 (segment (start 128.57 110.07) (end 127.1 108.6) (width 0.25) (layer B.Cu) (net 2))
 (segment (start 124.070001 121.400001) (end 124.92 122.25) (width 0.25) (layer B.Cu) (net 2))
 (segment (start 127.1 108.6) (end 124.15 108.6) (width 0.25) (layer B.Cu) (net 2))
 (segment (start 124.15 108.6) (end 121.700011 111.049989) (width 0.25) (layer B.Cu) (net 2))
 (segment (start 121.700011 119.030011) (end 124.070001 121.400001) (width 0.25) (layer B.Cu) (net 2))
 (segment (start 121.700011 111.049989) (end 121.700011 119.030011) (width 0.25) (layer B.Cu) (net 2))
 (segment (start 121.25 146.113589) (end 121.25 156.37) (width 0.25) (layer B.Cu) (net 3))
 (segment (start 121.25 156.37) (end 121.530001 156.650001) (width 0.25) (layer B.Cu) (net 3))
 (segment (start 127.050011 143.399989) (end 123.9636 143.399989) (width 0.25) (layer B.Cu) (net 3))
 (segment (start 121.530001 156.650001) (end 122.38 157.5) (width 0.25) (layer B.Cu) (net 3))
 (segment (start 129.61 140.84) (end 127.050011 143.399989) (width 0.25) (layer B.Cu) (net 3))
 (segment (start 131.16 140.84) (end 129.61 140.84) (width 0.25) (layer B.Cu) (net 3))
 (segment (start 123.9636 143.399989) (end 121.25 146.113589) (width 0.25) (layer B.Cu) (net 3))
 (segment (start 155.36 140.84) (end 152.800011 143.399989) (width 0.25) (layer B.Cu) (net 3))
 (segment (start 156.91 140.84) (end 155.36 140.84) (width 0.25) (layer B.Cu) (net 3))
 (segment (start 152.800011 143.399989) (end 149.7136 143.399989) (width 0.25) (layer B.Cu) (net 3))
 (segment (start 147 146.113589) (end 147 156.37) (width 0.25) (layer B.Cu) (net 3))
 (segment (start 147 156.37) (end 147.280001 156.650001) (width 0.25) (layer B.Cu) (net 3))
 (segment (start 147.280001 156.650001) (end 148.13 157.5) (width 0.25) (layer B.Cu) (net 3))
 (segment (start 149.7136 143.399989) (end 147 146.113589) (width 0.25) (layer B.Cu) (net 3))
 (segment (start 147 110.863589) (end 147 121.12) (width 0.25) (layer B.Cu) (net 3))
 (segment (start 152.800011 108.149989) (end 149.7136 108.149989) (width 0.25) (layer B.Cu) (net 3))
 (segment (start 149.7136 108.149989) (end 147 110.863589) (width 0.25) (layer B.Cu) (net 3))
 (segment (start 156.91 105.59) (end 155.36 105.59) (width 0.25) (layer B.Cu) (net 3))
 (segment (start 155.36 105.59) (end 152.800011 108.149989) (width 0.25) (layer B.Cu) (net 3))
 (segment (start 147.280001 121.400001) (end 148.13 122.25) (width 0.25) (layer B.Cu) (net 3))
 (segment (start 147 121.12) (end 147.280001 121.400001) (width 0.25) (layer B.Cu) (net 3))
 (segment (start 131.16 105.59) (end 129.61 105.59) (width 0.25) (layer B.Cu) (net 3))
 (segment (start 121.25 121.12) (end 121.530001 121.400001) (width 0.25) (layer B.Cu) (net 3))
 (segment (start 129.61 105.59) (end 127.050011 108.149989) (width 0.25) (layer B.Cu) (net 3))
 (segment (start 127.050011 108.149989) (end 123.9636 108.149989) (width 0.25) (layer B.Cu) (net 3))
 (segment (start 123.9636 108.149989) (end 121.25 110.863589) (width 0.25) (layer B.Cu) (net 3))
 (segment (start 121.25 110.863589) (end 121.25 121.12) (width 0.25) (layer B.Cu) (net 3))
 (segment (start 121.530001 121.400001) (end 122.38 122.25) (width 0.25) (layer B.Cu) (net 3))
 (segment (start 131.16 100.41) (end 127.09 100.41) (width 0.25) (layer B.Cu) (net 4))
 (segment (start 127.09 100.41) (end 116.5 111) (width 0.25) (layer B.Cu) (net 4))
 (segment (start 118.990001 121.400001) (end 119.84 122.25) (width 0.25) (layer B.Cu) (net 4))
 (segment (start 116.5 111) (end 116.5 118.91) (width 0.25) (layer B.Cu) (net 4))
 (segment (start 116.5 118.91) (end 118.990001 121.400001) (width 0.25) (layer B.Cu) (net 4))
 (segment (start 156.91 100.41) (end 152.84 100.41) (width 0.25) (layer B.Cu) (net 4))
 (segment (start 144.740001 121.400001) (end 145.59 122.25) (width 0.25) (layer B.Cu) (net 4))
 (segment (start 152.84 100.41) (end 142.25 111) (width 0.25) (layer B.Cu) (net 4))
 (segment (start 142.25 111) (end 142.25 118.91) (width 0.25) (layer B.Cu) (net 4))
 (segment (start 142.25 118.91) (end 144.740001 121.400001) (width 0.25) (layer B.Cu) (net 4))
 (segment (start 156.91 135.66) (end 152.84 135.66) (width 0.25) (layer B.Cu) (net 4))
 (segment (start 152.84 135.66) (end 142.25 146.25) (width 0.25) (layer B.Cu) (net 4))
 (segment (start 142.25 146.25) (end 142.25 154.16) (width 0.25) (layer B.Cu) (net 4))
 (segment (start 142.25 154.16) (end 144.740001 156.650001) (width 0.25) (layer B.Cu) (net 4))
 (segment (start 144.740001 156.650001) (end 145.59 157.5) (width 0.25) (layer B.Cu) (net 4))
 (segment (start 131.16 135.66) (end 127.09 135.66) (width 0.25) (layer B.Cu) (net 4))
 (segment (start 127.09 135.66) (end 116.5 146.25) (width 0.25) (layer B.Cu) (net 4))
 (segment (start 116.5 146.25) (end 116.5 154.16) (width 0.25) (layer B.Cu) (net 4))
 (segment (start 116.5 154.16) (end 118.990001 156.650001) (width 0.25) (layer B.Cu) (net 4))
 (segment (start 118.990001 156.650001) (end 119.84 157.5) (width 0.25) (layer B.Cu) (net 4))
 (segment (start 154.32 131.18) (end 143.75 141.75) (width 0.25) (layer B.Cu) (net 5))
 (segment (start 143.75 141.75) (end 139.75 141.75) (width 0.25) (layer B.Cu) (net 5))
 (segment (start 137.5 144) (end 137.5 150) (width 0.25) (layer B.Cu) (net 5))
 (segment (start 139.75 141.75) (end 137.5 144) (width 0.25) (layer B.Cu) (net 5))
 (segment (start 137.5 150) (end 140.51 153.01) (width 0.25) (layer B.Cu) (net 5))
 (segment (start 140.51 153.01) (end 140.51 157.5) (width 0.25) (layer B.Cu) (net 5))
 (segment (start 128.57 131.18) (end 118 141.75) (width 0.25) (layer B.Cu) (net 5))
 (segment (start 118 141.75) (end 114 141.75) (width 0.25) (layer B.Cu) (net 5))
 (segment (start 114 141.75) (end 111.75 144) (width 0.25) (layer B.Cu) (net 5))
 (segment (start 111.75 144) (end 111.75 150) (width 0.25) (layer B.Cu) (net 5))
 (segment (start 111.75 150) (end 114.76 153.01) (width 0.25) (layer B.Cu) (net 5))
 (segment (start 114.76 153.01) (end 114.76 157.5) (width 0.25) (layer B.Cu) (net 5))
 (segment (start 114.76 157.5) (end 115.962081 157.5) (width 0.25) (layer B.Cu) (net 5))
 (segment (start 115.962081 157.5) (end 117.3 157.5) (width 0.25) (layer B.Cu) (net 5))
 (segment (start 140.51 157.5) (end 141.712081 157.5) (width 0.25) (layer B.Cu) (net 5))
 (segment (start 141.712081 157.5) (end 143.05 157.5) (width 0.25) (layer B.Cu) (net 5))
 (segment (start 140.25 106.5) (end 137.5 109.25) (width 0.25) (layer B.Cu) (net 5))
 (segment (start 143.75 106.5) (end 140.25 106.5) (width 0.25) (layer B.Cu) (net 5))
 (segment (start 140.51 117.76) (end 140.51 122.25) (width 0.25) (layer B.Cu) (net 5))
 (segment (start 141.712081 122.25) (end 143.05 122.25) (width 0.25) (layer B.Cu) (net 5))
 (segment (start 140.51 122.25) (end 141.712081 122.25) (width 0.25) (layer B.Cu) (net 5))
 (segment (start 137.5 114.75) (end 140.51 117.76) (width 0.25) (layer B.Cu) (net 5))
 (segment (start 137.5 109.25) (end 137.5 114.75) (width 0.25) (layer B.Cu) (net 5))
 (segment (start 154.32 95.93) (end 143.75 106.5) (width 0.25) (layer B.Cu) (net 5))
 (segment (start 114.76 122.25) (end 115.962081 122.25) (width 0.25) (layer B.Cu) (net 5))
 (segment (start 115.962081 122.25) (end 117.3 122.25) (width 0.25) (layer B.Cu) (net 5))
 (segment (start 128.57 95.93) (end 118 106.5) (width 0.25) (layer B.Cu) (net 5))
 (segment (start 111.75 109.25) (end 111.75 114.75) (width 0.25) (layer B.Cu) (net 5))
 (segment (start 118 106.5) (end 114.5 106.5) (width 0.25) (layer B.Cu) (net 5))
 (segment (start 114.5 106.5) (end 111.75 109.25) (width 0.25) (layer B.Cu) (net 5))
 (segment (start 111.75 114.75) (end 114.76 117.76) (width 0.25) (layer B.Cu) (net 5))
 (segment (start 114.76 117.76) (end 114.76 122.25) (width 0.25) (layer B.Cu) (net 5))
 (segment (start 152.01 141) (end 147.5 141) (width 0.25) (layer F.Cu) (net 6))
 (segment (start 147.5 141) (end 137.97 150.53) (width 0.25) (layer F.Cu) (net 6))
 (segment (start 137.97 150.53) (end 137.97 156.297919) (width 0.25) (layer F.Cu) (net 6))
 (segment (start 137.97 156.297919) (end 137.97 157.5) (width 0.25) (layer F.Cu) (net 6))
 (segment (start 126.26 141) (end 121.75 141) (width 0.25) (layer F.Cu) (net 6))
 (segment (start 121.75 141) (end 112.22 150.53) (width 0.25) (layer F.Cu) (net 6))
 (segment (start 112.22 150.53) (end 112.22 156.297919) (width 0.25) (layer F.Cu) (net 6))
 (segment (start 112.22 156.297919) (end 112.22 157.5) (width 0.25) (layer F.Cu) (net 6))
 (segment (start 152.01 105.75) (end 148.25 105.75) (width 0.25) (layer F.Cu) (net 6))
 (segment (start 148.25 105.75) (end 137.97 116.03) (width 0.25) (layer F.Cu) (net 6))
 (segment (start 137.97 116.03) (end 137.97 121.047919) (width 0.25) (layer F.Cu) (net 6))
 (segment (start 137.97 121.047919) (end 137.97 122.25) (width 0.25) (layer F.Cu) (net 6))
 (segment (start 126.26 105.75) (end 122.25 105.75) (width 0.25) (layer F.Cu) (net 6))
 (segment (start 122.25 105.75) (end 112.22 115.78) (width 0.25) (layer F.Cu) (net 6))
 (segment (start 112.22 115.78) (end 112.22 121.047919) (width 0.25) (layer F.Cu) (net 6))
 (segment (start 112.22 121.047919) (end 112.22 122.25) (width 0.25) (layer F.Cu) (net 6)))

